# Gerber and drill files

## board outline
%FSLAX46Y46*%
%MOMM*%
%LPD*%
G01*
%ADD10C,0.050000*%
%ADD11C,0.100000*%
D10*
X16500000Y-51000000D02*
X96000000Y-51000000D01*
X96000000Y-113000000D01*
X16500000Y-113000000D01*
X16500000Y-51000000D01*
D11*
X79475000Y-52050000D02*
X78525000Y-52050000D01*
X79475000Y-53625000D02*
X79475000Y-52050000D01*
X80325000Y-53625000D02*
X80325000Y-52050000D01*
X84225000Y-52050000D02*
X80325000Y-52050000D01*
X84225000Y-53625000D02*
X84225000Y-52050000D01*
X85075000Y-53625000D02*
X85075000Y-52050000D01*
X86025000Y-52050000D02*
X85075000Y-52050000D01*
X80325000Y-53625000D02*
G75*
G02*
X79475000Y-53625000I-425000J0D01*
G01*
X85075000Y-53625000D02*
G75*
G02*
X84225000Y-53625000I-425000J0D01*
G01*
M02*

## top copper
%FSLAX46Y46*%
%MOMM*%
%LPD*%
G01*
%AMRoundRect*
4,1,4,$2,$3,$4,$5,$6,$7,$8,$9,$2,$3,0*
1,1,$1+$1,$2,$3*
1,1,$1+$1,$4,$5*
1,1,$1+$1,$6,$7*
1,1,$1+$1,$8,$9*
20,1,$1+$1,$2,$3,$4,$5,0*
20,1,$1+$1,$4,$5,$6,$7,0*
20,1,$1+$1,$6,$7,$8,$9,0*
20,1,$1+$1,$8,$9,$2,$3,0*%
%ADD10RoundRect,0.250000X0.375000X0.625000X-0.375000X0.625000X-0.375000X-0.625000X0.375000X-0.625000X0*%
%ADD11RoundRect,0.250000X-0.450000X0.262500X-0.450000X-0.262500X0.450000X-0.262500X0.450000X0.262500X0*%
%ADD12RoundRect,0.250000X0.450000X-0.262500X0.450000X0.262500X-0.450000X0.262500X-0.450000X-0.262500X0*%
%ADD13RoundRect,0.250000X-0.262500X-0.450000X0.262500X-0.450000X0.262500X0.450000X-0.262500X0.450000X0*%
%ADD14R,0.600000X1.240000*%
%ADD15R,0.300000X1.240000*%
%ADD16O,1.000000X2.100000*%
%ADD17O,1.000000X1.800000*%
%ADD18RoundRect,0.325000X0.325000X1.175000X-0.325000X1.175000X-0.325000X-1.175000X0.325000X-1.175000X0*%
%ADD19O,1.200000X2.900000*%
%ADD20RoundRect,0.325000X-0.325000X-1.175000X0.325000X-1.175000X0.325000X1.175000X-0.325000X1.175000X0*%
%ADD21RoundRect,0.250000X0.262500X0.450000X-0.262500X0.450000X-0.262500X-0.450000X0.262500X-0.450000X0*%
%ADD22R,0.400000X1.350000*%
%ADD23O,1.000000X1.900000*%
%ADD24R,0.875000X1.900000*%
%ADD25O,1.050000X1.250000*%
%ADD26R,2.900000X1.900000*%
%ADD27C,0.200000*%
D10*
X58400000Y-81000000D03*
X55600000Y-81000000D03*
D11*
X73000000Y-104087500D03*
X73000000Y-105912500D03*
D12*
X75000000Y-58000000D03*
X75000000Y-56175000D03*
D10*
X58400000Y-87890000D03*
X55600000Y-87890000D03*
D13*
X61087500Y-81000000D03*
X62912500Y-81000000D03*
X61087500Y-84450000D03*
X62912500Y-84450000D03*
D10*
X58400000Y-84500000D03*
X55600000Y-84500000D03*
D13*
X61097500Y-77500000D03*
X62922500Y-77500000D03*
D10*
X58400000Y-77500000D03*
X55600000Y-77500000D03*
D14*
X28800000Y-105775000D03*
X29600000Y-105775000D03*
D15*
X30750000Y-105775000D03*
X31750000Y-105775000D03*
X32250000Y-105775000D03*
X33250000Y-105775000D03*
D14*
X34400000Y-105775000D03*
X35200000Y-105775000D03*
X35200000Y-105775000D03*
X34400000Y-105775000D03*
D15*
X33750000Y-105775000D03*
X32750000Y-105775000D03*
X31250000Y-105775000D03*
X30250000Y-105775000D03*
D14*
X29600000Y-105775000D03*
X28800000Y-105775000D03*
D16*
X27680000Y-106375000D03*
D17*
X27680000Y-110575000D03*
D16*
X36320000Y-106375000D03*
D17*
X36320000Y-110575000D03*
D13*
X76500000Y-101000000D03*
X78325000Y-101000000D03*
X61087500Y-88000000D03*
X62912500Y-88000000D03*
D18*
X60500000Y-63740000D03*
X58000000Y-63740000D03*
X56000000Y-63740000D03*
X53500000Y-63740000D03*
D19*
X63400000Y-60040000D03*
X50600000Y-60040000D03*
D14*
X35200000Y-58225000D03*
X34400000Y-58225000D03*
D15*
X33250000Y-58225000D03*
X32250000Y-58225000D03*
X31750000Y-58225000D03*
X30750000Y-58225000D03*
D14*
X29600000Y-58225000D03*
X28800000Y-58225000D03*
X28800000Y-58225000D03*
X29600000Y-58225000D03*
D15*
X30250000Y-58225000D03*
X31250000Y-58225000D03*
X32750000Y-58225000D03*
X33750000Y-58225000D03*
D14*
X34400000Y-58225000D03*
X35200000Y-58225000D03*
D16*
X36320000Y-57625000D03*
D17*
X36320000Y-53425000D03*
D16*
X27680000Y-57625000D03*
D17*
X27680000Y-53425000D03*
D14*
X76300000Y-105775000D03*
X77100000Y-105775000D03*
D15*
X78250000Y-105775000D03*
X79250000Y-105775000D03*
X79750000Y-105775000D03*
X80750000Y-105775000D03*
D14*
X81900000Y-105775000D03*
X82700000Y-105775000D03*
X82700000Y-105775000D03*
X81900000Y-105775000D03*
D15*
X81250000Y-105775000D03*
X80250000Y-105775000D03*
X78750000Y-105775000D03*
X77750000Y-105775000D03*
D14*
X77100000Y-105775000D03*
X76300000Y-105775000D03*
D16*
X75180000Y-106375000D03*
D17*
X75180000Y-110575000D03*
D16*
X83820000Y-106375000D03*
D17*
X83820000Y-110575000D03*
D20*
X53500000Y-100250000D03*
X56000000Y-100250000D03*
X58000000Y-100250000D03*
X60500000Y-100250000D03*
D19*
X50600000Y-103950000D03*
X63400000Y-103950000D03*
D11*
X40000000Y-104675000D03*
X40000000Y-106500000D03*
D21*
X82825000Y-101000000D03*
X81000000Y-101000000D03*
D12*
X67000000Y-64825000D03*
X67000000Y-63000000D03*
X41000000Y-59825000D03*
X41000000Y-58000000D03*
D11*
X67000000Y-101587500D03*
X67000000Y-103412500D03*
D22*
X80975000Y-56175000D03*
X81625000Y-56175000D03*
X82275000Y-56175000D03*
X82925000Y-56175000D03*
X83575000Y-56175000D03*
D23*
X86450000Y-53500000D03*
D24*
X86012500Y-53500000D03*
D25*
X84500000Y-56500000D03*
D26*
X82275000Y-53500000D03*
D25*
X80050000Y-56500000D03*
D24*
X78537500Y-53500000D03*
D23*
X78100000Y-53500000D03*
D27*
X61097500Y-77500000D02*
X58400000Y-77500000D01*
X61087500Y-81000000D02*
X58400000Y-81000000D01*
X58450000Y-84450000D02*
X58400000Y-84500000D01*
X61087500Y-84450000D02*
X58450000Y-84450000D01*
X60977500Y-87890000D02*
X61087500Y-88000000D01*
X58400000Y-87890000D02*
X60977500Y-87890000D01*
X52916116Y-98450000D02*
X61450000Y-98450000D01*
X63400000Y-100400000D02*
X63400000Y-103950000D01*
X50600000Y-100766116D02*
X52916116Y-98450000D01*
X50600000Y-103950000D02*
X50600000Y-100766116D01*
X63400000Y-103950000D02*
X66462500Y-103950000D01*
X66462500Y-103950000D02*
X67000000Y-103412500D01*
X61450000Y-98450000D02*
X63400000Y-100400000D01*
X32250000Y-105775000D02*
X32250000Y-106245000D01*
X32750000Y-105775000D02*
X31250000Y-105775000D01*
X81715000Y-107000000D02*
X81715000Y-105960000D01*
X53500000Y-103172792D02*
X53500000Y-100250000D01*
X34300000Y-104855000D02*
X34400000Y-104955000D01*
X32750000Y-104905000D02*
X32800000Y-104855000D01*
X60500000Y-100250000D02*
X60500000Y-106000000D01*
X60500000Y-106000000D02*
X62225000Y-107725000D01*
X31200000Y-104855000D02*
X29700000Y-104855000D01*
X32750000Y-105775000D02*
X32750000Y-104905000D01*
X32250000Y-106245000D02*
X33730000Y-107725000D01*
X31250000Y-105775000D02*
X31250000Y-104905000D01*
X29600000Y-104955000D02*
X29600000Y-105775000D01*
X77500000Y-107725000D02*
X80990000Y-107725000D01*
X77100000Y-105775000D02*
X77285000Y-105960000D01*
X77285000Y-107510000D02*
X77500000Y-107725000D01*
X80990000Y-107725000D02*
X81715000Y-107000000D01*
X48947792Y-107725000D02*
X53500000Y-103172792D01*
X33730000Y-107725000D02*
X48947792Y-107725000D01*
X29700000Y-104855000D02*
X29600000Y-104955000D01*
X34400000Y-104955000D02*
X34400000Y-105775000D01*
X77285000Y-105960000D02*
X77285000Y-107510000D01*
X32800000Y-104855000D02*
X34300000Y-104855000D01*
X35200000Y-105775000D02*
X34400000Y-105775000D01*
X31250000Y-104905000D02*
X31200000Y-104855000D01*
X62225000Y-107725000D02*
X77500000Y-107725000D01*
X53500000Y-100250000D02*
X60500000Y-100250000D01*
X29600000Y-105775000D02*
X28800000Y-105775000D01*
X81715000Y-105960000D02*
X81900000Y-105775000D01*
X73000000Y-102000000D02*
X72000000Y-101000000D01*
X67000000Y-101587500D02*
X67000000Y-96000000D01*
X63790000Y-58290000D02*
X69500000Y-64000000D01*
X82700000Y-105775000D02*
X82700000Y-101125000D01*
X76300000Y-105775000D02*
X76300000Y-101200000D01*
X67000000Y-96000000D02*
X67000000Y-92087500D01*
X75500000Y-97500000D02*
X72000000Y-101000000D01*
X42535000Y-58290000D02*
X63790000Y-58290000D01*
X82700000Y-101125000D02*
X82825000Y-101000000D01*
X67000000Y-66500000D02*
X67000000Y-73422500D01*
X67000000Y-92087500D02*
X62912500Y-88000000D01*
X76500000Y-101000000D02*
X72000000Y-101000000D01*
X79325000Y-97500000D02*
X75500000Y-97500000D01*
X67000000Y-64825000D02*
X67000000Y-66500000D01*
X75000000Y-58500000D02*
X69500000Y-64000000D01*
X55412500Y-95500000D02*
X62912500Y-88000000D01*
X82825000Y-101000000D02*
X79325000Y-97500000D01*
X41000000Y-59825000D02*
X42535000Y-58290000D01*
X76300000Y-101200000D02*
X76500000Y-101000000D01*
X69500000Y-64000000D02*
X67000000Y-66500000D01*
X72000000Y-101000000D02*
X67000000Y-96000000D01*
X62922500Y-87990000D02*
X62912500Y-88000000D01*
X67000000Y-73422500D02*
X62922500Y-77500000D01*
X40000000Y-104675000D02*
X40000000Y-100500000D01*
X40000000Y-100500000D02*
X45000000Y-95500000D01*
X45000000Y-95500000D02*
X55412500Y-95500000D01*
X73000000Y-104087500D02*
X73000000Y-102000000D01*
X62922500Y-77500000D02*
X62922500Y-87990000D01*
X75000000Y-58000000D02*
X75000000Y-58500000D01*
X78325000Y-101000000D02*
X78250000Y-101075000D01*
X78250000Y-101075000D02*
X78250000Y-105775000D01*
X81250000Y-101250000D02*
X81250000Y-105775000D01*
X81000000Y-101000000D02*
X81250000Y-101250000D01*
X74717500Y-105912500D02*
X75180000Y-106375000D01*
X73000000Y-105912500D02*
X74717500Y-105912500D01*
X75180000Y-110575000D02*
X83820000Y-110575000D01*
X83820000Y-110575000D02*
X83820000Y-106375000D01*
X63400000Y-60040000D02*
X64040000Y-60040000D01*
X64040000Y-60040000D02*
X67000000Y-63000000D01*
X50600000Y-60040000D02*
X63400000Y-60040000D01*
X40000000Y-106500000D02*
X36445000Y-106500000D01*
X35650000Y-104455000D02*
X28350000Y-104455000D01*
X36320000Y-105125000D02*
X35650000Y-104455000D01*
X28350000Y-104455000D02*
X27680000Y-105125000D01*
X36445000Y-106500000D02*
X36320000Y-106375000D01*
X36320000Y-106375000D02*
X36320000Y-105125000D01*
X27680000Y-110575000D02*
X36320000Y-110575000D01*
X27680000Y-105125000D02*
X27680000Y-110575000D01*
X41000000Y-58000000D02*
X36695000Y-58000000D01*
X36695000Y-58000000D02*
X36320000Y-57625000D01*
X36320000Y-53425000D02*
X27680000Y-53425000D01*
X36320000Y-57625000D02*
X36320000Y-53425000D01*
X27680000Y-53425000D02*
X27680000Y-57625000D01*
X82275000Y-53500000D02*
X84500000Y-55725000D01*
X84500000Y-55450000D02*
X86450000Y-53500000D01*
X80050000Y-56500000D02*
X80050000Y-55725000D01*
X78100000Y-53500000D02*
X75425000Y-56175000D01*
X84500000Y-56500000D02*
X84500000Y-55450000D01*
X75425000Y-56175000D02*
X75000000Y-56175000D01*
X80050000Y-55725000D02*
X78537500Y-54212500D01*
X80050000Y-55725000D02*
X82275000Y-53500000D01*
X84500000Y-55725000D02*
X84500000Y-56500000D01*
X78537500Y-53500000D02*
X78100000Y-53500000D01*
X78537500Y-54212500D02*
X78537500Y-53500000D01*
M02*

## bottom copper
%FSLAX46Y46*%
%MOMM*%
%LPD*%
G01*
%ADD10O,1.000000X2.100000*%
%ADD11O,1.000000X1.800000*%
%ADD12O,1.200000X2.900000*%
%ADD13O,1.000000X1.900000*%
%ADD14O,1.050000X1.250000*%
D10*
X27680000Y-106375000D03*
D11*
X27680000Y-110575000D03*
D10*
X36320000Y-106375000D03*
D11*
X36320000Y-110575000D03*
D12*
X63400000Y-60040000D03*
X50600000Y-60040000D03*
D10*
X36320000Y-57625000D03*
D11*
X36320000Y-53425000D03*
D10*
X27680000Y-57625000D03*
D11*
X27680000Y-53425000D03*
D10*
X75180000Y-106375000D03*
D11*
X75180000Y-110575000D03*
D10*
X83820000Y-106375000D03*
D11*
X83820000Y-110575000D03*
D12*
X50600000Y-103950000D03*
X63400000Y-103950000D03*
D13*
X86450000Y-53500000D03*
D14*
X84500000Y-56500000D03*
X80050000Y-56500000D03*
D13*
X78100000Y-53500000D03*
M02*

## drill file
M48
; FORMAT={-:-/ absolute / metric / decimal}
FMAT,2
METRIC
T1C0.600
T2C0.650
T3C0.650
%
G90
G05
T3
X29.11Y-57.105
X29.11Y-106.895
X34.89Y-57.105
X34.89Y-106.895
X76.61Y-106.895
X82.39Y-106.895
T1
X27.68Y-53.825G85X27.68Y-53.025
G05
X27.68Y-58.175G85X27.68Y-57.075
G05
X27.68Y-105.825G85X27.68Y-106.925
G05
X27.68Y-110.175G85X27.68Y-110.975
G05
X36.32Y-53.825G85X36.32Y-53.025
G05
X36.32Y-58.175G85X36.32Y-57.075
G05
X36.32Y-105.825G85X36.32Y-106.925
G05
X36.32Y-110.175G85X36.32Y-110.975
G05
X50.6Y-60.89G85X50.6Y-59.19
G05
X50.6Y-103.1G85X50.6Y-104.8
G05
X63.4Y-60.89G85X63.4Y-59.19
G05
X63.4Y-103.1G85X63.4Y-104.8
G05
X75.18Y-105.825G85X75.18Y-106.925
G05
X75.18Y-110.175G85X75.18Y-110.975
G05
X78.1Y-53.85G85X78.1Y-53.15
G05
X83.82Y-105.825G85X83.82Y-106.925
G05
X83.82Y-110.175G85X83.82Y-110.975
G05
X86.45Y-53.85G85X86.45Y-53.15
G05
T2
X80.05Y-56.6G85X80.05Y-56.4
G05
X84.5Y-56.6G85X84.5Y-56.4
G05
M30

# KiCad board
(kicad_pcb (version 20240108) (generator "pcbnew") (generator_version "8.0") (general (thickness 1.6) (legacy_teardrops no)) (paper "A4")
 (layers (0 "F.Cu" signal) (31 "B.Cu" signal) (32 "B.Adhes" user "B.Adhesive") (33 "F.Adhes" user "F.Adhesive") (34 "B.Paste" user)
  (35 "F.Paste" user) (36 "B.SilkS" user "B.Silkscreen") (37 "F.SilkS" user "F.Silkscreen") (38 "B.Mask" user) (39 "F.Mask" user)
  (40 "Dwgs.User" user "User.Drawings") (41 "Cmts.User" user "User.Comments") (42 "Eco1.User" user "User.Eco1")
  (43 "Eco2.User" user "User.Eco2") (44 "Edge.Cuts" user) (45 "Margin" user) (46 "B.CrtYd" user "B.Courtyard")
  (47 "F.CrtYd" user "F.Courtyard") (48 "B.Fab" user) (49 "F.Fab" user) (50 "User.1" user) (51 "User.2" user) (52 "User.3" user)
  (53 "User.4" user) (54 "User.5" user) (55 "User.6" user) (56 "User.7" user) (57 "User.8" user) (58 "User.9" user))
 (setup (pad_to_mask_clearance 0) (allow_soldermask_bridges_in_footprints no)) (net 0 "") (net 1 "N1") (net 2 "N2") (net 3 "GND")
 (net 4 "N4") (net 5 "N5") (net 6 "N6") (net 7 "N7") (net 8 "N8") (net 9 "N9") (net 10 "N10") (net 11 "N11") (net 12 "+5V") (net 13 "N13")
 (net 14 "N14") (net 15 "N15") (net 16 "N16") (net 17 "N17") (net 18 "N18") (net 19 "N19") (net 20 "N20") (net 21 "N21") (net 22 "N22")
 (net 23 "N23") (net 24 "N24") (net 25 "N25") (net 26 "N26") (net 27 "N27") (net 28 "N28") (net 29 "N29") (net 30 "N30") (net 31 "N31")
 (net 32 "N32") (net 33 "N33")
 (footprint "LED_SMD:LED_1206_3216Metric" (layer "F.Cu") (at 57 81 180)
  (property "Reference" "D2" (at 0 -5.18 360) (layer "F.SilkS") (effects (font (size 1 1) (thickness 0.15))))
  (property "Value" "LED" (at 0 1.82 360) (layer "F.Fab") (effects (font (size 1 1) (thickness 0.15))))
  (pad "1" smd roundrect (at -1.4 0 180) (size 1.25 1.75) (layers "F.Cu" "F.Paste" "F.Mask") (roundrect_rratio 0.2) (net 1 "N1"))
  (pad "2" smd roundrect (at 1.4 0 180) (size 1.25 1.75) (layers "F.Cu" "F.Paste" "F.Mask") (roundrect_rratio 0.2) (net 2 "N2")))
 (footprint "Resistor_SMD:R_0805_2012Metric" (layer "F.Cu") (at 73 105 -90)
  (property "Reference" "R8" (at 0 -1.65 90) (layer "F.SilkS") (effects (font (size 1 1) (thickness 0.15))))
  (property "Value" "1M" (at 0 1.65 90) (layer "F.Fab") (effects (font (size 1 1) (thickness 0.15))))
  (pad "1" smd roundrect (at -0.9125 0 270) (size 1.025 1.4) (layers "F.Cu" "F.Paste" "F.Mask") (roundrect_rratio 0.243902) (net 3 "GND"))
  (pad "2" smd roundrect (at 0.9125 0 270) (size 1.025 1.4) (layers "F.Cu" "F.Paste" "F.Mask") (roundrect_rratio 0.243902) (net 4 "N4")))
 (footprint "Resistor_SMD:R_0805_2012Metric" (layer "F.Cu") (at 75 57.0875 90)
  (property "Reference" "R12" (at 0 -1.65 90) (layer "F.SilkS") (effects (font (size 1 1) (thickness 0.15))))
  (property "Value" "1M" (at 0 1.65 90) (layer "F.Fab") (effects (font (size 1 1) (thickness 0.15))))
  (pad "1" smd roundrect (at -0.9125 0 90) (size 1.025 1.4) (layers "F.Cu" "F.Paste" "F.Mask") (roundrect_rratio 0.243902) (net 3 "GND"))
  (pad "2" smd roundrect (at 0.9125 0 90) (size 1.025 1.4) (layers "F.Cu" "F.Paste" "F.Mask") (roundrect_rratio 0.243902) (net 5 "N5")))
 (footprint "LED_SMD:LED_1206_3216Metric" (layer "F.Cu") (at 57 87.89 180)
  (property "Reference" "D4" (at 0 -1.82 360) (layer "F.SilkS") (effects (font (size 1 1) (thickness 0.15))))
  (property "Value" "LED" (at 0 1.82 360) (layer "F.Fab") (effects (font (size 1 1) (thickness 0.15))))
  (pad "1" smd roundrect (at -1.4 0 180) (size 1.25 1.75) (layers "F.Cu" "F.Paste" "F.Mask") (roundrect_rratio 0.2) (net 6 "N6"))
  (pad "2" smd roundrect (at 1.4 0 180) (size 1.25 1.75) (layers "F.Cu" "F.Paste" "F.Mask") (roundrect_rratio 0.2) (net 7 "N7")))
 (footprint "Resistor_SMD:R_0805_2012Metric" (layer "F.Cu") (at 62 81)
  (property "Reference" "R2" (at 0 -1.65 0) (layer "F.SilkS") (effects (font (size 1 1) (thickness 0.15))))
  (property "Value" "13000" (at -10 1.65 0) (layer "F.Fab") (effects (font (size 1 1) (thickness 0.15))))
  (pad "1" smd roundrect (at -0.9125 0) (size 1.025 1.4) (layers "F.Cu" "F.Paste" "F.Mask") (roundrect_rratio 0.243902) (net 1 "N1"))
  (pad "2" smd roundrect (at 0.9125 0) (size 1.025 1.4) (layers "F.Cu" "F.Paste" "F.Mask") (roundrect_rratio 0.243902) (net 3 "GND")))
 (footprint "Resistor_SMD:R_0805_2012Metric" (layer "F.Cu") (at 62 84.45)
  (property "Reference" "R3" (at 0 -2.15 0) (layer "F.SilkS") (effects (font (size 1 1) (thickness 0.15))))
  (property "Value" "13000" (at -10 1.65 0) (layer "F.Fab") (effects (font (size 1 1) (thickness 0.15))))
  (pad "1" smd roundrect (at -0.9125 0) (size 1.025 1.4) (layers "F.Cu" "F.Paste" "F.Mask") (roundrect_rratio 0.243902) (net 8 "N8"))
  (pad "2" smd roundrect (at 0.9125 0) (size 1.025 1.4) (layers "F.Cu" "F.Paste" "F.Mask") (roundrect_rratio 0.243902) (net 3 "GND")))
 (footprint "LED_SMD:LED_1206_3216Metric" (layer "F.Cu") (at 57 84.5 180)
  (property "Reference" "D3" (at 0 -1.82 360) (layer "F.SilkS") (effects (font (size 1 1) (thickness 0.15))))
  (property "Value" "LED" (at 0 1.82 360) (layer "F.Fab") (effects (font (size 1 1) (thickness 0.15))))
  (pad "1" smd roundrect (at -1.4 0 180) (size 1.25 1.75) (layers "F.Cu" "F.Paste" "F.Mask") (roundrect_rratio 0.2) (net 8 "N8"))
  (pad "2" smd roundrect (at 1.4 0 180) (size 1.25 1.75) (layers "F.Cu" "F.Paste" "F.Mask") (roundrect_rratio 0.2) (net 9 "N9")))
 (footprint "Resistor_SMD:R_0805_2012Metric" (layer "F.Cu") (at 62.01 77.5)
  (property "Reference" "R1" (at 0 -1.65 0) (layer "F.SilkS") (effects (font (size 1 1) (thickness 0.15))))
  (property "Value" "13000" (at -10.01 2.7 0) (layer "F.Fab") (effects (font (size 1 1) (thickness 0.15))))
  (pad "1" smd roundrect (at -0.9125 0) (size 1.025 1.4) (layers "F.Cu" "F.Paste" "F.Mask") (roundrect_rratio 0.243902) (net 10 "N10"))
  (pad "2" smd roundrect (at 0.9125 0) (size 1.025 1.4) (layers "F.Cu" "F.Paste" "F.Mask") (roundrect_rratio 0.243902) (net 3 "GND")))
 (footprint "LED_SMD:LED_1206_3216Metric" (layer "F.Cu") (at 57 77.5 180)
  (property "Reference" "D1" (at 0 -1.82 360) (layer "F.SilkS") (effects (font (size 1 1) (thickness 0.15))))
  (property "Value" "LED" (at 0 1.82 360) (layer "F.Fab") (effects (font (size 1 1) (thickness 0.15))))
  (pad "1" smd roundrect (at -1.4 0 180) (size 1.25 1.75) (layers "F.Cu" "F.Paste" "F.Mask") (roundrect_rratio 0.2) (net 10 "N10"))
  (pad "2" smd roundrect (at 1.4 0 180) (size 1.25 1.75) (layers "F.Cu" "F.Paste" "F.Mask") (roundrect_rratio 0.2) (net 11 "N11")))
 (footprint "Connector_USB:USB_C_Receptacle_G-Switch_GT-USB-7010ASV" (layer "F.Cu") (at 32 109.5)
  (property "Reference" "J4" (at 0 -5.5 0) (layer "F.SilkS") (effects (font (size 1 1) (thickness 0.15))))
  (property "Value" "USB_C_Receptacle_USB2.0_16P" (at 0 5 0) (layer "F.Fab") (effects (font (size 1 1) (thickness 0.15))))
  (pad "" np_thru_hole circle (at -2.89 -2.605) (size 0.65 0.65) (drill 0.65) (layers "*.Cu" "*.Mask"))
  (pad "" np_thru_hole circle (at 2.89 -2.605) (size 0.65 0.65) (drill 0.65) (layers "*.Cu" "*.Mask"))
  (pad "A1" smd rect (at -3.2 -3.725) (size 0.6 1.24) (layers "F.Cu" "F.Paste" "F.Mask") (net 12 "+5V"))
  (pad "A4" smd rect (at -2.4 -3.725) (size 0.6 1.24) (layers "F.Cu" "F.Paste" "F.Mask") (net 12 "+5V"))
  (pad "A5" smd rect (at -1.25 -3.725) (size 0.3 1.24) (layers "F.Cu" "F.Paste" "F.Mask") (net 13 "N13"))
  (pad "A6" smd rect (at -0.25 -3.725) (size 0.3 1.24) (layers "F.Cu" "F.Paste" "F.Mask") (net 12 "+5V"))
  (pad "A7" smd rect (at 0.25 -3.725) (size 0.3 1.24) (layers "F.Cu" "F.Paste" "F.Mask") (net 12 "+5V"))
  (pad "A8" smd rect (at 1.25 -3.725) (size 0.3 1.24) (layers "F.Cu" "F.Paste" "F.Mask") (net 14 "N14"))
  (pad "A9" smd rect (at 2.4 -3.725) (size 0.6 1.24) (layers "F.Cu" "F.Paste" "F.Mask") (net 12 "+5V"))
  (pad "A12" smd rect (at 3.2 -3.725) (size 0.6 1.24) (layers "F.Cu" "F.Paste" "F.Mask") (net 12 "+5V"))
  (pad "B1" smd rect (at 3.2 -3.725) (size 0.6 1.24) (layers "F.Cu" "F.Paste" "F.Mask") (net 12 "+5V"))
  (pad "B4" smd rect (at 2.4 -3.725) (size 0.6 1.24) (layers "F.Cu" "F.Paste" "F.Mask") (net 12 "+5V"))
  (pad "B5" smd rect (at 1.75 -3.725) (size 0.3 1.24) (layers "F.Cu" "F.Paste" "F.Mask") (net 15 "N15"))
  (pad "B6" smd rect (at 0.75 -3.725) (size 0.3 1.24) (layers "F.Cu" "F.Paste" "F.Mask") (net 12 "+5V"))
  (pad "B7" smd rect (at -0.75 -3.725) (size 0.3 1.24) (layers "F.Cu" "F.Paste" "F.Mask") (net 12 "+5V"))
  (pad "B8" smd rect (at -1.75 -3.725) (size 0.3 1.24) (layers "F.Cu" "F.Paste" "F.Mask") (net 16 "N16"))
  (pad "B9" smd rect (at -2.4 -3.725) (size 0.6 1.24) (layers "F.Cu" "F.Paste" "F.Mask") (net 12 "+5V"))
  (pad "B12" smd rect (at -3.2 -3.725) (size 0.6 1.24) (layers "F.Cu" "F.Paste" "F.Mask") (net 12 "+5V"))
  (pad "S1" thru_hole oval (at -4.32 -3.125) (size 1 2.1) (drill oval 0.6 1.7) (layers "*.Cu" "*.Mask") (remove_unused_layers no)
   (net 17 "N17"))
  (pad "S1" thru_hole oval (at -4.32 1.075) (size 1 1.8) (drill oval 0.6 1.4) (layers "*.Cu" "*.Mask") (remove_unused_layers no)
   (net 17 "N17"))
  (pad "S1" thru_hole oval (at 4.32 -3.125) (size 1 2.1) (drill oval 0.6 1.7) (layers "*.Cu" "*.Mask") (remove_unused_layers no)
   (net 17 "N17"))
  (pad "S1" thru_hole oval (at 4.32 1.075) (size 1 1.8) (drill oval 0.6 1.4) (layers "*.Cu" "*.Mask") (remove_unused_layers no)
   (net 17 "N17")))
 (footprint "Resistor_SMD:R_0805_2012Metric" (layer "F.Cu") (at 77.4125 101)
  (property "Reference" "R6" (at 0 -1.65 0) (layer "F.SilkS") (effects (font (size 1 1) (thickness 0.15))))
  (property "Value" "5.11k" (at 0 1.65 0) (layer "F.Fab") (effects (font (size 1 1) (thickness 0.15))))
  (pad "1" smd roundrect (at -0.9125 0) (size 1.025 1.4) (layers "F.Cu" "F.Paste" "F.Mask") (roundrect_rratio 0.243902) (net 3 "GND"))
  (pad "2" smd roundrect (at 0.9125 0) (size 1.025 1.4) (layers "F.Cu" "F.Paste" "F.Mask") (roundrect_rratio 0.243902) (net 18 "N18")))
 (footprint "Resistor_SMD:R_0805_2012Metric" (layer "F.Cu") (at 62 88)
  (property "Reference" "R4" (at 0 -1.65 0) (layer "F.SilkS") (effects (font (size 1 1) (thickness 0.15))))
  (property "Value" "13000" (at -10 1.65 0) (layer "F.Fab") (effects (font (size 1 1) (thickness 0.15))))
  (pad "1" smd roundrect (at -0.9125 0) (size 1.025 1.4) (layers "F.Cu" "F.Paste" "F.Mask") (roundrect_rratio 0.243902) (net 6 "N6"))
  (pad "2" smd roundrect (at 0.9125 0) (size 1.025 1.4) (layers "F.Cu" "F.Paste" "F.Mask") (roundrect_rratio 0.243902) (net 3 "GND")))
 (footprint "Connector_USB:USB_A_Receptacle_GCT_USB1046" (layer "F.Cu") (at 57 56.49 180)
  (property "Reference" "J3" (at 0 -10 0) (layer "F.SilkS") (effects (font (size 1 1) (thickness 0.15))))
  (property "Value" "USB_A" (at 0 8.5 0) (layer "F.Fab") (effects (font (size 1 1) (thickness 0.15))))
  (pad "" smd oval (at -6.4 -3.55 180) (size 1.2 2.9) (layers "F.Paste") (thermal_bridge_angle 45))
  (pad "" smd oval (at 6.4 -3.55 180) (size 1.2 2.9) (layers "F.Paste") (thermal_bridge_angle 45))
  (pad "1" smd roundrect (at -3.5 -7.25 180) (size 1.3 3) (layers "F.Cu" "F.Paste" "F.Mask") (roundrect_rratio 0.25) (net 11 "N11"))
  (pad "2" smd roundrect (at -1 -7.25 180) (size 1.3 3) (layers "F.Cu" "F.Paste" "F.Mask") (roundrect_rratio 0.25) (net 9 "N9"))
  (pad "3" smd roundrect (at 1 -7.25 180) (size 1.3 3) (layers "F.Cu" "F.Paste" "F.Mask") (roundrect_rratio 0.25) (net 2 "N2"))
  (pad "4" smd roundrect (at 3.5 -7.25 180) (size 1.3 3) (layers "F.Cu" "F.Paste" "F.Mask") (roundrect_rratio 0.25) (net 7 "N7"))
  (pad "5" thru_hole oval (at -6.4 -3.55 180) (size 1.2 2.9) (drill oval 0.6 2.3) (layers "*.Cu" "*.Mask") (remove_unused_layers no)
   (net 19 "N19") (thermal_bridge_angle 45))
  (pad "5" thru_hole oval (at 6.4 -3.55 180) (size 1.2 2.9) (drill oval 0.6 2.3) (layers "*.Cu" "*.Mask") (remove_unused_layers no)
   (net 19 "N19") (thermal_bridge_angle 45)))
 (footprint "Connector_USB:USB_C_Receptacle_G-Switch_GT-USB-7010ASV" (layer "F.Cu") (at 32 54.5 180)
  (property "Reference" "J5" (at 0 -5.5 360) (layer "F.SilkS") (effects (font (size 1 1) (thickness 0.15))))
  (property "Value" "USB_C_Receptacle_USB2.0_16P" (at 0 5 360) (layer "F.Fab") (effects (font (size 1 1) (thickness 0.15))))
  (pad "" np_thru_hole circle (at -2.89 -2.605 180) (size 0.65 0.65) (drill 0.65) (layers "*.Cu" "*.Mask"))
  (pad "" np_thru_hole circle (at 2.89 -2.605 180) (size 0.65 0.65) (drill 0.65) (layers "*.Cu" "*.Mask"))
  (pad "A1" smd rect (at -3.2 -3.725 180) (size 0.6 1.24) (layers "F.Cu" "F.Paste" "F.Mask") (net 7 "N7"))
  (pad "A4" smd rect (at -2.4 -3.725 180) (size 0.6 1.24) (layers "F.Cu" "F.Paste" "F.Mask") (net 11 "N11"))
  (pad "A5" smd rect (at -1.25 -3.725 180) (size 0.3 1.24) (layers "F.Cu" "F.Paste" "F.Mask") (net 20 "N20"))
  (pad "A6" smd rect (at -0.25 -3.725 180) (size 0.3 1.24) (layers "F.Cu" "F.Paste" "F.Mask") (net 2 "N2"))
  (pad "A7" smd rect (at 0.25 -3.725 180) (size 0.3 1.24) (layers "F.Cu" "F.Paste" "F.Mask") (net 9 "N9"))
  (pad "A8" smd rect (at 1.25 -3.725 180) (size 0.3 1.24) (layers "F.Cu" "F.Paste" "F.Mask") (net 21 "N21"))
  (pad "A9" smd rect (at 2.4 -3.725 180) (size 0.6 1.24) (layers "F.Cu" "F.Paste" "F.Mask") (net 11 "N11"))
  (pad "A12" smd rect (at 3.2 -3.725 180) (size 0.6 1.24) (layers "F.Cu" "F.Paste" "F.Mask") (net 7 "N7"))
  (pad "B1" smd rect (at 3.2 -3.725 180) (size 0.6 1.24) (layers "F.Cu" "F.Paste" "F.Mask") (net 7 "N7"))
  (pad "B4" smd rect (at 2.4 -3.725 180) (size 0.6 1.24) (layers "F.Cu" "F.Paste" "F.Mask") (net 11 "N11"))
  (pad "B5" smd rect (at 1.75 -3.725 180) (size 0.3 1.24) (layers "F.Cu" "F.Paste" "F.Mask") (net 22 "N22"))
  (pad "B6" smd rect (at 0.75 -3.725 180) (size 0.3 1.24) (layers "F.Cu" "F.Paste" "F.Mask") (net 2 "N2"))
  (pad "B7" smd rect (at -0.75 -3.725 180) (size 0.3 1.24) (layers "F.Cu" "F.Paste" "F.Mask") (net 9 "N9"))
  (pad "B8" smd rect (at -1.75 -3.725 180) (size 0.3 1.24) (layers "F.Cu" "F.Paste" "F.Mask") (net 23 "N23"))
  (pad "B9" smd rect (at -2.4 -3.725 180) (size 0.6 1.24) (layers "F.Cu" "F.Paste" "F.Mask") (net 11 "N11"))
  (pad "B12" smd rect (at -3.2 -3.725 180) (size 0.6 1.24) (layers "F.Cu" "F.Paste" "F.Mask") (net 7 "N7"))
  (pad "S1" thru_hole oval (at -4.32 -3.125 180) (size 1 2.1) (drill oval 0.6 1.7) (layers "*.Cu" "*.Mask") (remove_unused_layers no)
   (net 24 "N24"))
  (pad "S1" thru_hole oval (at -4.32 1.075 180) (size 1 1.8) (drill oval 0.6 1.4) (layers "*.Cu" "*.Mask") (remove_unused_layers no)
   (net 24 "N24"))
  (pad "S1" thru_hole oval (at 4.32 -3.125 180) (size 1 2.1) (drill oval 0.6 1.7) (layers "*.Cu" "*.Mask") (remove_unused_layers no)
   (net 24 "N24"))
  (pad "S1" thru_hole oval (at 4.32 1.075 180) (size 1 1.8) (drill oval 0.6 1.4) (layers "*.Cu" "*.Mask") (remove_unused_layers no)
   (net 24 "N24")))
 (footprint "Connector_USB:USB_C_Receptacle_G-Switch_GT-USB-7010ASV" (layer "F.Cu") (at 79.5 109.5)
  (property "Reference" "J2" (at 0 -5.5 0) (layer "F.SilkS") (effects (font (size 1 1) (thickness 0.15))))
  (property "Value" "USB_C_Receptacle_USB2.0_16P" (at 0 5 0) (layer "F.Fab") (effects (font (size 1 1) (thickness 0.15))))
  (pad "" np_thru_hole circle (at -2.89 -2.605) (size 0.65 0.65) (drill 0.65) (layers "*.Cu" "*.Mask"))
  (pad "" np_thru_hole circle (at 2.89 -2.605) (size 0.65 0.65) (drill 0.65) (layers "*.Cu" "*.Mask"))
  (pad "A1" smd rect (at -3.2 -3.725) (size 0.6 1.24) (layers "F.Cu" "F.Paste" "F.Mask") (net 3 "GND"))
  (pad "A4" smd rect (at -2.4 -3.725) (size 0.6 1.24) (layers "F.Cu" "F.Paste" "F.Mask") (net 12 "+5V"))
  (pad "A5" smd rect (at -1.25 -3.725) (size 0.3 1.24) (layers "F.Cu" "F.Paste" "F.Mask") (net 18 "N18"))
  (pad "A6" smd rect (at -0.25 -3.725) (size 0.3 1.24) (layers "F.Cu" "F.Paste" "F.Mask") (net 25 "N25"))
  (pad "A7" smd rect (at 0.25 -3.725) (size 0.3 1.24) (layers "F.Cu" "F.Paste" "F.Mask") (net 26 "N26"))
  (pad "A8" smd rect (at 1.25 -3.725) (size 0.3 1.24) (layers "F.Cu" "F.Paste" "F.Mask") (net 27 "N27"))
  (pad "A9" smd rect (at 2.4 -3.725) (size 0.6 1.24) (layers "F.Cu" "F.Paste" "F.Mask") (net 12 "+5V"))
  (pad "A12" smd rect (at 3.2 -3.725) (size 0.6 1.24) (layers "F.Cu" "F.Paste" "F.Mask") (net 3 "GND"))
  (pad "B1" smd rect (at 3.2 -3.725) (size 0.6 1.24) (layers "F.Cu" "F.Paste" "F.Mask") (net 3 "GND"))
  (pad "B4" smd rect (at 2.4 -3.725) (size 0.6 1.24) (layers "F.Cu" "F.Paste" "F.Mask") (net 12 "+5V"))
  (pad "B5" smd rect (at 1.75 -3.725) (size 0.3 1.24) (layers "F.Cu" "F.Paste" "F.Mask") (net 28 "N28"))
  (pad "B6" smd rect (at 0.75 -3.725) (size 0.3 1.24) (layers "F.Cu" "F.Paste" "F.Mask") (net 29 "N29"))
  (pad "B7" smd rect (at -0.75 -3.725) (size 0.3 1.24) (layers "F.Cu" "F.Paste" "F.Mask") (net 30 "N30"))
  (pad "B8" smd rect (at -1.75 -3.725) (size 0.3 1.24) (layers "F.Cu" "F.Paste" "F.Mask") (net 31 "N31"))
  (pad "B9" smd rect (at -2.4 -3.725) (size 0.6 1.24) (layers "F.Cu" "F.Paste" "F.Mask") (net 12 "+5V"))
  (pad "B12" smd rect (at -3.2 -3.725) (size 0.6 1.24) (layers "F.Cu" "F.Paste" "F.Mask") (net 3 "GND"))
  (pad "S1" thru_hole oval (at -4.32 -3.125) (size 1 2.1) (drill oval 0.6 1.7) (layers "*.Cu" "*.Mask") (remove_unused_layers no)
   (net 4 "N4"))
  (pad "S1" thru_hole oval (at -4.32 1.075) (size 1 1.8) (drill oval 0.6 1.4) (layers "*.Cu" "*.Mask") (remove_unused_layers no)
   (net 4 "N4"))
  (pad "S1" thru_hole oval (at 4.32 -3.125) (size 1 2.1) (drill oval 0.6 1.7) (layers "*.Cu" "*.Mask") (remove_unused_layers no)
   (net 4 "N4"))
  (pad "S1" thru_hole oval (at 4.32 1.075) (size 1 1.8) (drill oval 0.6 1.4) (layers "*.Cu" "*.Mask") (remove_unused_layers no) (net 4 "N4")))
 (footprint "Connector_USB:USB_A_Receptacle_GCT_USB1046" (layer "F.Cu") (at 57 107.5)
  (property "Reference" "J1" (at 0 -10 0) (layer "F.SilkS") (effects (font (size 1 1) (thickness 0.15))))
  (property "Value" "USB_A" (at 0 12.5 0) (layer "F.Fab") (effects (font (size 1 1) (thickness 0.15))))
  (pad "" smd oval (at -6.4 -3.55) (size 1.2 2.9) (layers "F.Paste") (thermal_bridge_angle 45))
  (pad "" smd oval (at 6.4 -3.55) (size 1.2 2.9) (layers "F.Paste") (thermal_bridge_angle 45))
  (pad "1" smd roundrect (at -3.5 -7.25) (size 1.3 3) (layers "F.Cu" "F.Paste" "F.Mask") (roundrect_rratio 0.25) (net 12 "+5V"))
  (pad "2" smd roundrect (at -1 -7.25) (size 1.3 3) (layers "F.Cu" "F.Paste" "F.Mask") (roundrect_rratio 0.25) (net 12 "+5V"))
  (pad "3" smd roundrect (at 1 -7.25) (size 1.3 3) (layers "F.Cu" "F.Paste" "F.Mask") (roundrect_rratio 0.25) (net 12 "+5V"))
  (pad "4" smd roundrect (at 3.5 -7.25) (size 1.3 3) (layers "F.Cu" "F.Paste" "F.Mask") (roundrect_rratio 0.25) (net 12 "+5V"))
  (pad "5" thru_hole oval (at -6.4 -3.55) (size 1.2 2.9) (drill oval 0.6 2.3) (layers "*.Cu" "*.Mask") (remove_unused_layers no)
   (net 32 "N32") (thermal_bridge_angle 45))
  (pad "5" thru_hole oval (at 6.4 -3.55) (size 1.2 2.9) (drill oval 0.6 2.3) (layers "*.Cu" "*.Mask") (remove_unused_layers no)
   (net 32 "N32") (thermal_bridge_angle 45)))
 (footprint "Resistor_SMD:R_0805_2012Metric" (layer "F.Cu") (at 40 105.5875 -90)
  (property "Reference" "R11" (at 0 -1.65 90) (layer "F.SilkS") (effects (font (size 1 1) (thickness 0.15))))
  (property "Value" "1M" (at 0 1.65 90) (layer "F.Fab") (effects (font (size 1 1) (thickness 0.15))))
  (pad "1" smd roundrect (at -0.9125 0 270) (size 1.025 1.4) (layers "F.Cu" "F.Paste" "F.Mask") (roundrect_rratio 0.243902) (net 3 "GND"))
  (pad "2" smd roundrect (at 0.9125 0 270) (size 1.025 1.4) (layers "F.Cu" "F.Paste" "F.Mask") (roundrect_rratio 0.243902) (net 17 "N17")))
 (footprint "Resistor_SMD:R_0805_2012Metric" (layer "F.Cu") (at 81.9125 101 180)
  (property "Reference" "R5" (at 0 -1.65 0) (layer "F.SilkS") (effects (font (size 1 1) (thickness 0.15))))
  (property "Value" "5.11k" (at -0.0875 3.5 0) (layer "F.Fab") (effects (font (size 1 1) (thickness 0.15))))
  (pad "1" smd roundrect (at -0.9125 0 180) (size 1.025 1.4) (layers "F.Cu" "F.Paste" "F.Mask") (roundrect_rratio 0.243902) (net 3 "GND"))
  (pad "2" smd roundrect (at 0.9125 0 180) (size 1.025 1.4) (layers "F.Cu" "F.Paste" "F.Mask") (roundrect_rratio 0.243902) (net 28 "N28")))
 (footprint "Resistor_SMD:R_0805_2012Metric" (layer "F.Cu") (at 67 63.9125 90)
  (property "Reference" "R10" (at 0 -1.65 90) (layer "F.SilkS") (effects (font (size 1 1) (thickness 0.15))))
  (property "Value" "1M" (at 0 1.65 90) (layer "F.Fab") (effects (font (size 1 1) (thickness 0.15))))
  (pad "1" smd roundrect (at -0.9125 0 90) (size 1.025 1.4) (layers "F.Cu" "F.Paste" "F.Mask") (roundrect_rratio 0.243902) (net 3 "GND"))
  (pad "2" smd roundrect (at 0.9125 0 90) (size 1.025 1.4) (layers "F.Cu" "F.Paste" "F.Mask") (roundrect_rratio 0.243902) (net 19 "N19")))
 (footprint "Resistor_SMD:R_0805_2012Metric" (layer "F.Cu") (at 41 58.9125 90)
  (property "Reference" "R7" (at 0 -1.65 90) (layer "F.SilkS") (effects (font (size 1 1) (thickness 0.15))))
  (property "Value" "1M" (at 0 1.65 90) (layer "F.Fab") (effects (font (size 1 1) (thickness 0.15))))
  (pad "1" smd roundrect (at -0.9125 0 90) (size 1.025 1.4) (layers "F.Cu" "F.Paste" "F.Mask") (roundrect_rratio 0.243902) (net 3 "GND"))
  (pad "2" smd roundrect (at 0.9125 0 90) (size 1.025 1.4) (layers "F.Cu" "F.Paste" "F.Mask") (roundrect_rratio 0.243902) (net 24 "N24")))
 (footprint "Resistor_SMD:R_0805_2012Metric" (layer "F.Cu") (at 67 102.5 -90)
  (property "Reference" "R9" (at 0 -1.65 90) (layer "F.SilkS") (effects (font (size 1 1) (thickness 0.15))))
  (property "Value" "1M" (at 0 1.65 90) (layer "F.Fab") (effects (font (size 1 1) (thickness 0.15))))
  (pad "1" smd roundrect (at -0.9125 0 270) (size 1.025 1.4) (layers "F.Cu" "F.Paste" "F.Mask") (roundrect_rratio 0.243902) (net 3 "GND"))
  (pad "2" smd roundrect (at 0.9125 0 270) (size 1.025 1.4) (layers "F.Cu" "F.Paste" "F.Mask") (roundrect_rratio 0.243902) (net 32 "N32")))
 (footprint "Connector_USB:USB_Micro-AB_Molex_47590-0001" (layer "F.Cu") (at 82.275 53.5 180)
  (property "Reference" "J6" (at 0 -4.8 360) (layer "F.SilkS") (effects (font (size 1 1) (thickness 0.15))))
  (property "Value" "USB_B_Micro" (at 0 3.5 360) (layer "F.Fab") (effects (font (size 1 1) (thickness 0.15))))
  (fp_line (start 2.8 1.45) (end 3.75 1.45) (stroke (width 0.1) (type solid)) (layer "Edge.Cuts"))
  (fp_line (start 2.8 -0.125) (end 2.8 1.45) (stroke (width 0.1) (type solid)) (layer "Edge.Cuts"))
  (fp_line (start 1.95 -0.125) (end 1.95 1.45) (stroke (width 0.1) (type solid)) (layer "Edge.Cuts"))
  (fp_line (start -1.95 1.45) (end 1.95 1.45) (stroke (width 0.1) (type solid)) (layer "Edge.Cuts"))
  (fp_line (start -1.95 -0.125) (end -1.95 1.45) (stroke (width 0.1) (type solid)) (layer "Edge.Cuts"))
  (fp_line (start -2.8 -0.125) (end -2.8 1.45) (stroke (width 0.1) (type solid)) (layer "Edge.Cuts"))
  (fp_line (start -3.75 1.45) (end -2.8 1.45) (stroke (width 0.1) (type solid)) (layer "Edge.Cuts"))
  (fp_arc (start 1.95 -0.125) (mid 2.375 -0.55) (end 2.8 -0.125) (stroke (width 0.1) (type solid)) (layer "Edge.Cuts"))
  (fp_arc (start -2.8 -0.125) (mid -2.375 -0.55) (end -1.95 -0.125) (stroke (width 0.1) (type solid)) (layer "Edge.Cuts"))
  (pad "" smd rect (at -3.5 0 180) (size 0.3 0.85) (layers "F.Paste"))
  (pad "" smd rect (at 3.5 0 180) (size 0.3 0.85) (layers "F.Paste"))
  (pad "1" smd rect (at 1.3 -2.675 180) (size 0.4 1.35) (layers "F.Cu" "F.Paste" "F.Mask") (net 11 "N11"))
  (pad "2" smd rect (at 0.65 -2.675 180) (size 0.4 1.35) (layers "F.Cu" "F.Paste" "F.Mask") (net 9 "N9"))
  (pad "3" smd rect (at 0 -2.675 180) (size 0.4 1.35) (layers "F.Cu" "F.Paste" "F.Mask") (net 2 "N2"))
  (pad "4" smd rect (at -0.65 -2.675 180) (size 0.4 1.35) (layers "F.Cu" "F.Paste" "F.Mask") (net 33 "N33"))
  (pad "5" smd rect (at -1.3 -2.675 180) (size 0.4 1.35) (layers "F.Cu" "F.Paste" "F.Mask") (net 7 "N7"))
  (pad "6" thru_hole oval (at -4.175 0 180) (size 1 1.9) (drill oval 0.6 1.3) (layers "*.Cu" "*.Mask") (remove_unused_layers no)
   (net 5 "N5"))
  (pad "6" smd rect (at -3.7375 0 180) (size 0.875 1.9) (layers "F.Cu" "F.Mask") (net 5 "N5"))
  (pad "6" thru_hole oval (at -2.225 -3 180) (size 1.05 1.25) (drill oval 0.65 0.85) (layers "*.Cu" "*.Mask") (remove_unused_layers no)
   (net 5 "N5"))
  (pad "6" smd rect (at 0 0 180) (size 2.9 1.9) (layers "F.Cu" "F.Paste" "F.Mask") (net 5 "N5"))
  (pad "6" thru_hole oval (at 2.225 -3 180) (size 1.05 1.25) (drill oval 0.65 0.85) (layers "*.Cu" "*.Mask") (remove_unused_layers no)
   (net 5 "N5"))
  (pad "6" smd rect (at 3.7375 0 180) (size 0.875 1.9) (layers "F.Cu" "F.Mask") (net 5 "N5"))
  (pad "6" thru_hole oval (at 4.175 0 180) (size 1 1.9) (drill oval 0.6 1.3) (layers "*.Cu" "*.Mask") (remove_unused_layers no) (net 5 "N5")))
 (gr_rect (start 16.5 51) (end 96 113) (stroke (width 0.05) (type default)) (fill none) (layer "Edge.Cuts"))
 (segment (start 61.0975 77.5) (end 58.4 77.5) (width 0.2) (layer "F.Cu") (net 10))
 (segment (start 61.0875 81) (end 58.4 81) (width 0.2) (layer "F.Cu") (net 1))
 (segment (start 58.45 84.45) (end 58.4 84.5) (width 0.2) (layer "F.Cu") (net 8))
 (segment (start 61.0875 84.45) (end 58.45 84.45) (width 0.2) (layer "F.Cu") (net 8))
 (segment (start 60.9775 87.89) (end 61.0875 88) (width 0.2) (layer "F.Cu") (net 6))
 (segment (start 58.4 87.89) (end 60.9775 87.89) (width 0.2) (layer "F.Cu") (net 6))
 (segment (start 52.916116 98.45) (end 61.45 98.45) (width 0.2) (layer "F.Cu") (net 32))
 (segment (start 63.4 100.4) (end 63.4 103.95) (width 0.2) (layer "F.Cu") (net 32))
 (segment (start 50.6 100.766116) (end 52.916116 98.45) (width 0.2) (layer "F.Cu") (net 32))
 (segment (start 50.6 103.95) (end 50.6 100.766116) (width 0.2) (layer "F.Cu") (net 32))
 (segment (start 63.4 103.95) (end 66.4625 103.95) (width 0.2) (layer "F.Cu") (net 32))
 (segment (start 66.4625 103.95) (end 67 103.4125) (width 0.2) (layer "F.Cu") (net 32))
 (segment (start 61.45 98.45) (end 63.4 100.4) (width 0.2) (layer "F.Cu") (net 32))
 (segment (start 32.25 105.775) (end 32.25 106.245) (width 0.2) (layer "F.Cu") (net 12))
 (segment (start 32.75 105.775) (end 31.25 105.775) (width 0.2) (layer "F.Cu") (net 12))
 (segment (start 81.715 107) (end 81.715 105.96) (width 0.2) (layer "F.Cu") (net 12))
 (segment (start 53.5 103.172792) (end 53.5 100.25) (width 0.2) (layer "F.Cu") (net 12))
 (segment (start 34.3 104.855) (end 34.4 104.955) (width 0.2) (layer "F.Cu") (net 12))
 (segment (start 32.75 104.905) (end 32.8 104.855) (width 0.2) (layer "F.Cu") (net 12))
 (segment (start 60.5 100.25) (end 60.5 106) (width 0.2) (layer "F.Cu") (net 12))
 (segment (start 60.5 106) (end 62.225 107.725) (width 0.2) (layer "F.Cu") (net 12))
 (segment (start 31.2 104.855) (end 29.7 104.855) (width 0.2) (layer "F.Cu") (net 12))
 (segment (start 32.75 105.775) (end 32.75 104.905) (width 0.2) (layer "F.Cu") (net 12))
 (segment (start 32.25 106.245) (end 33.73 107.725) (width 0.2) (layer "F.Cu") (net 12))
 (segment (start 31.25 105.775) (end 31.25 104.905) (width 0.2) (layer "F.Cu") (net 12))
 (segment (start 29.6 104.955) (end 29.6 105.775) (width 0.2) (layer "F.Cu") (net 12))
 (segment (start 77.5 107.725) (end 80.99 107.725) (width 0.2) (layer "F.Cu") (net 12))
 (segment (start 77.1 105.775) (end 77.285 105.96) (width 0.2) (layer "F.Cu") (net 12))
 (segment (start 77.285 107.51) (end 77.5 107.725) (width 0.2) (layer "F.Cu") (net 12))
 (segment (start 80.99 107.725) (end 81.715 107) (width 0.2) (layer "F.Cu") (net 12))
 (segment (start 48.947792 107.725) (end 53.5 103.172792) (width 0.2) (layer "F.Cu") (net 12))
 (segment (start 33.73 107.725) (end 48.947792 107.725) (width 0.2) (layer "F.Cu") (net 12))
 (segment (start 29.7 104.855) (end 29.6 104.955) (width 0.2) (layer "F.Cu") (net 12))
 (segment (start 34.4 104.955) (end 34.4 105.775) (width 0.2) (layer "F.Cu") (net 12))
 (segment (start 77.285 105.96) (end 77.285 107.51) (width 0.2) (layer "F.Cu") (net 12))
 (segment (start 32.8 104.855) (end 34.3 104.855) (width 0.2) (layer "F.Cu") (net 12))
 (segment (start 35.2 105.775) (end 34.4 105.775) (width 0.2) (layer "F.Cu") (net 12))
 (segment (start 31.25 104.905) (end 31.2 104.855) (width 0.2) (layer "F.Cu") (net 12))
 (segment (start 62.225 107.725) (end 77.5 107.725) (width 0.2) (layer "F.Cu") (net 12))
 (segment (start 53.5 100.25) (end 60.5 100.25) (width 0.2) (layer "F.Cu") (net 12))
 (segment (start 29.6 105.775) (end 28.8 105.775) (width 0.2) (layer "F.Cu") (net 12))
 (segment (start 81.715 105.96) (end 81.9 105.775) (width 0.2) (layer "F.Cu") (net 12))
 (segment (start 73 102) (end 72 101) (width 0.2) (layer "F.Cu") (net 3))
 (segment (start 67 101.5875) (end 67 96) (width 0.2) (layer "F.Cu") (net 3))
 (segment (start 63.79 58.29) (end 69.5 64) (width 0.2) (layer "F.Cu") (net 3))
 (segment (start 82.7 105.775) (end 82.7 101.125) (width 0.2) (layer "F.Cu") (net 3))
 (segment (start 76.3 105.775) (end 76.3 101.2) (width 0.2) (layer "F.Cu") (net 3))
 (segment (start 67 96) (end 67 92.0875) (width 0.2) (layer "F.Cu") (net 3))
 (segment (start 75.5 97.5) (end 72 101) (width 0.2) (layer "F.Cu") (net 3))
 (segment (start 42.535 58.29) (end 63.79 58.29) (width 0.2) (layer "F.Cu") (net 3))
 (segment (start 82.7 101.125) (end 82.825 101) (width 0.2) (layer "F.Cu") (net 3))
 (segment (start 67 66.5) (end 67 73.4225) (width 0.2) (layer "F.Cu") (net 3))
 (segment (start 67 92.0875) (end 62.9125 88) (width 0.2) (layer "F.Cu") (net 3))
 (segment (start 76.5 101) (end 72 101) (width 0.2) (layer "F.Cu") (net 3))
 (segment (start 79.325 97.5) (end 75.5 97.5) (width 0.2) (layer "F.Cu") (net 3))
 (segment (start 67 64.825) (end 67 66.5) (width 0.2) (layer "F.Cu") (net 3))
 (segment (start 75 58.5) (end 69.5 64) (width 0.2) (layer "F.Cu") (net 3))
 (segment (start 55.4125 95.5) (end 62.9125 88) (width 0.2) (layer "F.Cu") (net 3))
 (segment (start 82.825 101) (end 79.325 97.5) (width 0.2) (layer "F.Cu") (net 3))
 (segment (start 41 59.825) (end 42.535 58.29) (width 0.2) (layer "F.Cu") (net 3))
 (segment (start 76.3 101.2) (end 76.5 101) (width 0.2) (layer "F.Cu") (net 3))
 (segment (start 69.5 64) (end 67 66.5) (width 0.2) (layer "F.Cu") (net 3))
 (segment (start 72 101) (end 67 96) (width 0.2) (layer "F.Cu") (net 3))
 (segment (start 62.9225 87.99) (end 62.9125 88) (width 0.2) (layer "F.Cu") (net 3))
 (segment (start 67 73.4225) (end 62.9225 77.5) (width 0.2) (layer "F.Cu") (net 3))
 (segment (start 40 104.675) (end 40 100.5) (width 0.2) (layer "F.Cu") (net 3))
 (segment (start 40 100.5) (end 45 95.5) (width 0.2) (layer "F.Cu") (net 3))
 (segment (start 45 95.5) (end 55.4125 95.5) (width 0.2) (layer "F.Cu") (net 3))
 (segment (start 73 104.0875) (end 73 102) (width 0.2) (layer "F.Cu") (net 3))
 (segment (start 62.9225 77.5) (end 62.9225 87.99) (width 0.2) (layer "F.Cu") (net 3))
 (segment (start 75 58) (end 75 58.5) (width 0.2) (layer "F.Cu") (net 3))
 (segment (start 78.325 101) (end 78.25 101.075) (width 0.2) (layer "F.Cu") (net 18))
 (segment (start 78.25 101.075) (end 78.25 105.775) (width 0.2) (layer "F.Cu") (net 18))
 (segment (start 81.25 101.25) (end 81.25 105.775) (width 0.2) (layer "F.Cu") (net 28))
 (segment (start 81 101) (end 81.25 101.25) (width 0.2) (layer "F.Cu") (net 28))
 (segment (start 74.7175 105.9125) (end 75.18 106.375) (width 0.2) (layer "F.Cu") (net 4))
 (segment (start 73 105.9125) (end 74.7175 105.9125) (width 0.2) (layer "F.Cu") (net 4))
 (segment (start 75.18 110.575) (end 83.82 110.575) (width 0.2) (layer "F.Cu") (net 4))
 (segment (start 83.82 110.575) (end 83.82 106.375) (width 0.2) (layer "F.Cu") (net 4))
 (segment (start 63.4 60.04) (end 64.04 60.04) (width 0.2) (layer "F.Cu") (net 19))
 (segment (start 64.04 60.04) (end 67 63) (width 0.2) (layer "F.Cu") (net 19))
 (segment (start 50.6 60.04) (end 63.4 60.04) (width 0.2) (layer "F.Cu") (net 19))
 (segment (start 40 106.5) (end 36.445 106.5) (width 0.2) (layer "F.Cu") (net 17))
 (segment (start 35.65 104.455) (end 28.35 104.455) (width 0.2) (layer "F.Cu") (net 17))
 (segment (start 36.32 105.125) (end 35.65 104.455) (width 0.2) (layer "F.Cu") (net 17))
 (segment (start 28.35 104.455) (end 27.68 105.125) (width 0.2) (layer "F.Cu") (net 17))
 (segment (start 36.445 106.5) (end 36.32 106.375) (width 0.2) (layer "F.Cu") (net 17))
 (segment (start 36.32 106.375) (end 36.32 105.125) (width 0.2) (layer "F.Cu") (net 17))
 (segment (start 27.68 110.575) (end 36.32 110.575) (width 0.2) (layer "F.Cu") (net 17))
 (segment (start 27.68 105.125) (end 27.68 110.575) (width 0.2) (layer "F.Cu") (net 17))
 (segment (start 41 58) (end 36.695 58) (width 0.2) (layer "F.Cu") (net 24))
 (segment (start 36.695 58) (end 36.32 57.625) (width 0.2) (layer "F.Cu") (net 24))
 (segment (start 36.32 53.425) (end 27.68 53.425) (width 0.2) (layer "F.Cu") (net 24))
 (segment (start 36.32 57.625) (end 36.32 53.425) (width 0.2) (layer "F.Cu") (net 24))
 (segment (start 27.68 53.425) (end 27.68 57.625) (width 0.2) (layer "F.Cu") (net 24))
 (segment (start 82.275 53.5) (end 84.5 55.725) (width 0.2) (layer "F.Cu") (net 5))
 (segment (start 84.5 55.45) (end 86.45 53.5) (width 0.2) (layer "F.Cu") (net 5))
 (segment (start 80.05 56.5) (end 80.05 55.725) (width 0.2) (layer "F.Cu") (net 5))
 (segment (start 78.1 53.5) (end 75.425 56.175) (width 0.2) (layer "F.Cu") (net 5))
 (segment (start 84.5 56.5) (end 84.5 55.45) (width 0.2) (layer "F.Cu") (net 5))
 (segment (start 75.425 56.175) (end 75 56.175) (width 0.2) (layer "F.Cu") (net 5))
 (segment (start 80.05 55.725) (end 78.5375 54.2125) (width 0.2) (layer "F.Cu") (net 5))
 (segment (start 80.05 55.725) (end 82.275 53.5) (width 0.2) (layer "F.Cu") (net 5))
 (segment (start 84.5 55.725) (end 84.5 56.5) (width 0.2) (layer "F.Cu") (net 5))
 (segment (start 78.5375 53.5) (end 78.1 53.5) (width 0.2) (layer "F.Cu") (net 5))
 (segment (start 78.5375 54.2125) (end 78.5375 53.5) (width 0.2) (layer "F.Cu") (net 5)))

